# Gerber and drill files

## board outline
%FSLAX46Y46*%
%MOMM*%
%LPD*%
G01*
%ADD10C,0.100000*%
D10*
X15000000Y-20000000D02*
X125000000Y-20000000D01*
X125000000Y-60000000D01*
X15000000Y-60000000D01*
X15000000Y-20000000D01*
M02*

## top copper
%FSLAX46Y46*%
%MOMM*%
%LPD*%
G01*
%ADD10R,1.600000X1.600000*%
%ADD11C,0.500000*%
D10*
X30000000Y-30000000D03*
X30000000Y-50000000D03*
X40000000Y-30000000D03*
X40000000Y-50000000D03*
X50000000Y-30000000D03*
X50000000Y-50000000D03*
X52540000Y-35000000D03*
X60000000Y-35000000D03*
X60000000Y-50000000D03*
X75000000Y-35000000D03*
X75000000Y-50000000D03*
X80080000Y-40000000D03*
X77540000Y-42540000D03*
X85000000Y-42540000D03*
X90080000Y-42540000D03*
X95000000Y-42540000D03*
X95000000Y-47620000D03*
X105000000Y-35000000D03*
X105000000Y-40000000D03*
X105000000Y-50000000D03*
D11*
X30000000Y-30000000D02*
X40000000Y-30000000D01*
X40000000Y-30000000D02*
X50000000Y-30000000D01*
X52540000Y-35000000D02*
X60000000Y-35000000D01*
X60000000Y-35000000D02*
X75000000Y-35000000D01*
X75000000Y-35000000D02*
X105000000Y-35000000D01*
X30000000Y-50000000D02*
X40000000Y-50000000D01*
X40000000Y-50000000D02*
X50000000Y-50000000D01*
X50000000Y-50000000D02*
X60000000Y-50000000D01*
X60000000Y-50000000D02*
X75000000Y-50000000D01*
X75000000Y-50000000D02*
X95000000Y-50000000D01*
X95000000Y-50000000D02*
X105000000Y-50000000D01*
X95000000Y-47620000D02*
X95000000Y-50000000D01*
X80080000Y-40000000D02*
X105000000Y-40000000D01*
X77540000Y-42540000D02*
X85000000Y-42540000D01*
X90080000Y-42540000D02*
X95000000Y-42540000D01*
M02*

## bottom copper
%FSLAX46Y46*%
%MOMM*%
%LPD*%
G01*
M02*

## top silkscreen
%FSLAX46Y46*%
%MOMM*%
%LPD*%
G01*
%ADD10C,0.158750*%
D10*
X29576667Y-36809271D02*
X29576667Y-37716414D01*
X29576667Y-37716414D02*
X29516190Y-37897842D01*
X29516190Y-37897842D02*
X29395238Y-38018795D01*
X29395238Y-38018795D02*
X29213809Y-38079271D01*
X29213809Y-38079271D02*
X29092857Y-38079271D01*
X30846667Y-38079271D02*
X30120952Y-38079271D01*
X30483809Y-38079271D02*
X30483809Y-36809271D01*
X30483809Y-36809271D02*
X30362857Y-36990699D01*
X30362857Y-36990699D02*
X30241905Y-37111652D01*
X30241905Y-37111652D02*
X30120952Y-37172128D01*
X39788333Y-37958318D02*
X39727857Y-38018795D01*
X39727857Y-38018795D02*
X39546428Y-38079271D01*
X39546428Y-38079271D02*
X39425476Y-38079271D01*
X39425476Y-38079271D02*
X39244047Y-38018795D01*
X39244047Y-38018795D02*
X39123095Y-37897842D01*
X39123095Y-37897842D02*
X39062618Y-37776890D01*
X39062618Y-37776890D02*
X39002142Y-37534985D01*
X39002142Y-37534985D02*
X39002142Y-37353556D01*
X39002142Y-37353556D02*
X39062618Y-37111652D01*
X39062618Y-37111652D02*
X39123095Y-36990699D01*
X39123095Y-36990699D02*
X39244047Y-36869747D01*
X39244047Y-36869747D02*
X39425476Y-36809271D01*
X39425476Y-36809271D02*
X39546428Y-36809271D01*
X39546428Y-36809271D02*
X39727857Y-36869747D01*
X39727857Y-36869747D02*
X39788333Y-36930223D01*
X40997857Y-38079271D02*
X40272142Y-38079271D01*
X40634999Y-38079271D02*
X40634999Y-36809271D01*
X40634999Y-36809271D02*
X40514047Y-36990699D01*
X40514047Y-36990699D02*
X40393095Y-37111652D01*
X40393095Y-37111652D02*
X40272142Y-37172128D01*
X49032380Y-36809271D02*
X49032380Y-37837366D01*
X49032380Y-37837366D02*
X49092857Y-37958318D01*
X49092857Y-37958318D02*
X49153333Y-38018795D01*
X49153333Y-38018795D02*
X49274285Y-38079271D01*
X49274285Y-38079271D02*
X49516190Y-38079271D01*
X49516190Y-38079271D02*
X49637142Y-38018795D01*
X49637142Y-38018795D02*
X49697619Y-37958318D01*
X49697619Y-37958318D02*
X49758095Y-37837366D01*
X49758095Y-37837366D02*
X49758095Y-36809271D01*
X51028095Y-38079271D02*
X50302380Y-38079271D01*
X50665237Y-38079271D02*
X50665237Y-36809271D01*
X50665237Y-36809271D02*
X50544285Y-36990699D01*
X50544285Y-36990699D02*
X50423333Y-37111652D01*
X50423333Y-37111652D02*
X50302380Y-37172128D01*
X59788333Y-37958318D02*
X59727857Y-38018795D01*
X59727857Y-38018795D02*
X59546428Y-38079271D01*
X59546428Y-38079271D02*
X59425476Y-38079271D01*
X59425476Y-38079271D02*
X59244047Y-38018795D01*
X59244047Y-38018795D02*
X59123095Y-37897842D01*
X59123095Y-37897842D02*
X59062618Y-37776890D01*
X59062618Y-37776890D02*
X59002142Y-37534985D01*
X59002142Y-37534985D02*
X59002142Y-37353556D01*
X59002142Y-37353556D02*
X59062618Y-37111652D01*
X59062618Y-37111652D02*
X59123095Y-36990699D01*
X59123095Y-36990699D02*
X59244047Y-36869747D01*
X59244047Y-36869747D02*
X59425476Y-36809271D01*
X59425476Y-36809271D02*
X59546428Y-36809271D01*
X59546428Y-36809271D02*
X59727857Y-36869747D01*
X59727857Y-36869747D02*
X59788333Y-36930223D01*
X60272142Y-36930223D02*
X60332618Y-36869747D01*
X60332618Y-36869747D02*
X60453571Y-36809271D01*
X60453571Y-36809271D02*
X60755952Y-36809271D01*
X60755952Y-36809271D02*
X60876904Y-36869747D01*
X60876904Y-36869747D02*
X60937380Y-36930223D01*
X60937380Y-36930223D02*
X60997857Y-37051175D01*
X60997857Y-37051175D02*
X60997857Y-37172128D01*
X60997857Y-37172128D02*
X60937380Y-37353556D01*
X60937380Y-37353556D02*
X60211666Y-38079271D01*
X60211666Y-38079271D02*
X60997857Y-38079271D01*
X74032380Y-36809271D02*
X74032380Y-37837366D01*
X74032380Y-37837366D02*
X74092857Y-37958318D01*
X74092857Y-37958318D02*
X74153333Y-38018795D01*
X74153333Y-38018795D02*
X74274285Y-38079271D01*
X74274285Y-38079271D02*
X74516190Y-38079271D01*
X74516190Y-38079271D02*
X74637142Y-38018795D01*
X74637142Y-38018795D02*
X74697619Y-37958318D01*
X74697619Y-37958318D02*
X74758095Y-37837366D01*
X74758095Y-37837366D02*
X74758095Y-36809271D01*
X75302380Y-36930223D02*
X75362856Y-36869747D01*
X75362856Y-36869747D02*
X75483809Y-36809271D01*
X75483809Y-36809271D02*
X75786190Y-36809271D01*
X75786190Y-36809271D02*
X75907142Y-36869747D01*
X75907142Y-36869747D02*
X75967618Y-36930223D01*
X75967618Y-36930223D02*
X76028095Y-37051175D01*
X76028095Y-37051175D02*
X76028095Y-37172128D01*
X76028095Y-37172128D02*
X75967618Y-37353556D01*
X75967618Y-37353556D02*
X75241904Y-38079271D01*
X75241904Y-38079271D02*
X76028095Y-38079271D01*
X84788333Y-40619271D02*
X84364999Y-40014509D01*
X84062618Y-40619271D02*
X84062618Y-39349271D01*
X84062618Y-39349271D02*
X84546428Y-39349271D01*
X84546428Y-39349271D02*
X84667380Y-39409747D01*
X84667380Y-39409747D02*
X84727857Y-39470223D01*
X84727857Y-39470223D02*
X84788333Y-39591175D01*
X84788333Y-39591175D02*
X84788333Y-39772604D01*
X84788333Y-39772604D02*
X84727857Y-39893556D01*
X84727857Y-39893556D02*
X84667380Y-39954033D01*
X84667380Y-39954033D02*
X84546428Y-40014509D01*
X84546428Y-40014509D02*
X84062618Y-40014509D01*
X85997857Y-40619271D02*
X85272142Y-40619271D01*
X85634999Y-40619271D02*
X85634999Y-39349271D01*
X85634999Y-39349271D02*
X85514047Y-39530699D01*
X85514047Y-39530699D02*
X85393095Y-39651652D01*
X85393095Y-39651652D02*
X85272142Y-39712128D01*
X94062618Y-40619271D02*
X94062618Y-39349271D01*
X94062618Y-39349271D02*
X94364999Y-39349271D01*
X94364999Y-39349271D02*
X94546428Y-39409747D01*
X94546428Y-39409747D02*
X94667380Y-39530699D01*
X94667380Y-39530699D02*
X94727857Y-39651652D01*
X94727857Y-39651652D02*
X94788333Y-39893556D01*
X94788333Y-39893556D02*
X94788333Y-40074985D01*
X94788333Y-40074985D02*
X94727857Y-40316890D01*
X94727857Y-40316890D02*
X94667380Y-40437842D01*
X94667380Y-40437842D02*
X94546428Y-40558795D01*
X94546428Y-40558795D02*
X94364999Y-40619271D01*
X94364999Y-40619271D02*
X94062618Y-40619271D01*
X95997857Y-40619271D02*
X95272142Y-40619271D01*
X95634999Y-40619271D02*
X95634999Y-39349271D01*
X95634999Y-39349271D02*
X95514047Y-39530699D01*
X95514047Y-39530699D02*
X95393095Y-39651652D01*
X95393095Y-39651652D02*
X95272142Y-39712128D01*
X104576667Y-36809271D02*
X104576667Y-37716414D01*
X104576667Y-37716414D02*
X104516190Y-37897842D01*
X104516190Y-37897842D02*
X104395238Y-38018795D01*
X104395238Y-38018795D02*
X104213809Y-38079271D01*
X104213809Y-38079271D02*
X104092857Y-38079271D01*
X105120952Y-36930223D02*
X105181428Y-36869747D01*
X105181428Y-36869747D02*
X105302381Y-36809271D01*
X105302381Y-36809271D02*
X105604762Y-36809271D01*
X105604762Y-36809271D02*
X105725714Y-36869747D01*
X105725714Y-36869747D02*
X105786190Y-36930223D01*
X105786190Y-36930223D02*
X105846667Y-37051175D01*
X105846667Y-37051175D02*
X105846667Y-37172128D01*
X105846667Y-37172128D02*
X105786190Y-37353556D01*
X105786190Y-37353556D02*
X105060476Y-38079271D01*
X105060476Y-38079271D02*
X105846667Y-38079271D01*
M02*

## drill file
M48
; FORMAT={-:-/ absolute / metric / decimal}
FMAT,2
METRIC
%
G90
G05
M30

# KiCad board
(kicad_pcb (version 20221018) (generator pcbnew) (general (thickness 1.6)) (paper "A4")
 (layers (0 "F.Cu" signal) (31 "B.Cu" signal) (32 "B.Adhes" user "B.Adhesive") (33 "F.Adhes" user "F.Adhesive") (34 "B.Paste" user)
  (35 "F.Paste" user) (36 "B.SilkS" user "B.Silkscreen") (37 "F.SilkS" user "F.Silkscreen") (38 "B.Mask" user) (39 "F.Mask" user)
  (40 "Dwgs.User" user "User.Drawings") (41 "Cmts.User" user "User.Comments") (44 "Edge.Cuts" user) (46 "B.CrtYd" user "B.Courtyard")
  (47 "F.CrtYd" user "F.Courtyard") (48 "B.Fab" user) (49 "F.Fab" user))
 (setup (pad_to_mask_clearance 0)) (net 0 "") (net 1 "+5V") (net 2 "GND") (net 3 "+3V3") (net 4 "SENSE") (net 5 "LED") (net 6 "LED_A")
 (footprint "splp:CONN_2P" (layer "F.Cu") (at 30 40)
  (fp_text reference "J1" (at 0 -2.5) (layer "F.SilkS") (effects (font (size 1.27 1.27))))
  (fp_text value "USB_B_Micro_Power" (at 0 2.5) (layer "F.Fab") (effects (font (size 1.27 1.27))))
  (pad "1" smd rect (at 0 -10) (size 1.6 1.6) (layers "F.Cu" "F.Paste" "F.Mask") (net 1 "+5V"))
  (pad "2" smd rect (at 0 10) (size 1.6 1.6) (layers "F.Cu" "F.Paste" "F.Mask") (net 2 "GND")))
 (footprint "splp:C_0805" (layer "F.Cu") (at 40 40)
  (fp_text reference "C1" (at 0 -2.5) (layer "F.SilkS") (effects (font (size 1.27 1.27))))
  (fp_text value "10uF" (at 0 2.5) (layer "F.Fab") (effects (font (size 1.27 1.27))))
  (pad "1" smd rect (at 0 -10) (size 1.6 1.6) (layers "F.Cu" "F.Paste" "F.Mask") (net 1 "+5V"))
  (pad "2" smd rect (at 0 10) (size 1.6 1.6) (layers "F.Cu" "F.Paste" "F.Mask") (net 2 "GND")))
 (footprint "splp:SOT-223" (layer "F.Cu") (at 50 40)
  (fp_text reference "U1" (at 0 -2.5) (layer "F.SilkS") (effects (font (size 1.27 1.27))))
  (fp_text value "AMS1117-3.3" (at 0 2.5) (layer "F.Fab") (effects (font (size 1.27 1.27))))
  (pad "1" smd rect (at 0 -10) (size 1.6 1.6) (layers "F.Cu" "F.Paste" "F.Mask") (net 1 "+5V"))
  (pad "2" smd rect (at 0 10) (size 1.6 1.6) (layers "F.Cu" "F.Paste" "F.Mask") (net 2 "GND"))
  (pad "3" smd rect (at 2.54 -5) (size 1.6 1.6) (layers "F.Cu" "F.Paste" "F.Mask") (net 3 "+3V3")))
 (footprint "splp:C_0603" (layer "F.Cu") (at 60 40)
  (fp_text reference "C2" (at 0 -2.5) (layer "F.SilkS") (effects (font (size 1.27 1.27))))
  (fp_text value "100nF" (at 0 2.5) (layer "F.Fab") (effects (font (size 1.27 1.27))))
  (pad "1" smd rect (at 0 -5) (size 1.6 1.6) (layers "F.Cu" "F.Paste" "F.Mask") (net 3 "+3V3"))
  (pad "2" smd rect (at 0 10) (size 1.6 1.6) (layers "F.Cu" "F.Paste" "F.Mask") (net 2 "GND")))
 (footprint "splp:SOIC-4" (layer "F.Cu") (at 75 40)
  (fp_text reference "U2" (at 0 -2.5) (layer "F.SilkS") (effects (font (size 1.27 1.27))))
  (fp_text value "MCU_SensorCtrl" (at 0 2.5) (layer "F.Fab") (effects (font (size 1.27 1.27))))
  (pad "1" smd rect (at 0 -5) (size 1.6 1.6) (layers "F.Cu" "F.Paste" "F.Mask") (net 3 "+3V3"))
  (pad "2" smd rect (at 0 10) (size 1.6 1.6) (layers "F.Cu" "F.Paste" "F.Mask") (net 2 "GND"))
  (pad "3" smd rect (at 5.08 0) (size 1.6 1.6) (layers "F.Cu" "F.Paste" "F.Mask") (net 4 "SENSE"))
  (pad "4" smd rect (at 2.54 2.54) (size 1.6 1.6) (layers "F.Cu" "F.Paste" "F.Mask") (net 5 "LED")))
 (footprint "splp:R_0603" (layer "F.Cu") (at 85 42.54)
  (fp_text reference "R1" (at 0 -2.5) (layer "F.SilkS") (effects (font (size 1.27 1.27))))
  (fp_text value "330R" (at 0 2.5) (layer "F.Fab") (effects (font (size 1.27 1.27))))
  (pad "1" smd rect (at 0 0) (size 1.6 1.6) (layers "F.Cu" "F.Paste" "F.Mask") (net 5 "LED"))
  (pad "2" smd rect (at 5.08 0) (size 1.6 1.6) (layers "F.Cu" "F.Paste" "F.Mask") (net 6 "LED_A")))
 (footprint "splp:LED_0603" (layer "F.Cu") (at 95 42.54)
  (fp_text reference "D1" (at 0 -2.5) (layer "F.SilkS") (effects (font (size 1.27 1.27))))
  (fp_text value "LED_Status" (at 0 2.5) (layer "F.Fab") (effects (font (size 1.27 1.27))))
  (pad "1" smd rect (at 0 0) (size 1.6 1.6) (layers "F.Cu" "F.Paste" "F.Mask") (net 6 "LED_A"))
  (pad "2" smd rect (at 0 5.08) (size 1.6 1.6) (layers "F.Cu" "F.Paste" "F.Mask") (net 2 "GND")))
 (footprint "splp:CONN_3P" (layer "F.Cu") (at 105 40)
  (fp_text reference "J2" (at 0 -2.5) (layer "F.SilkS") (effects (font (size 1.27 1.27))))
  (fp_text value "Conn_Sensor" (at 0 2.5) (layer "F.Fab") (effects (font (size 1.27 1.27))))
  (pad "1" smd rect (at 0 -5) (size 1.6 1.6) (layers "F.Cu" "F.Paste" "F.Mask") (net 3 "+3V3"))
  (pad "2" smd rect (at 0 0) (size 1.6 1.6) (layers "F.Cu" "F.Paste" "F.Mask") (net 4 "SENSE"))
  (pad "3" smd rect (at 0 10) (size 1.6 1.6) (layers "F.Cu" "F.Paste" "F.Mask") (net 2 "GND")))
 (segment (start 30 30) (end 40 30) (width 0.5) (layer "F.Cu") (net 1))
 (segment (start 40 30) (end 50 30) (width 0.5) (layer "F.Cu") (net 1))
 (segment (start 52.54 35) (end 60 35) (width 0.5) (layer "F.Cu") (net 3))
 (segment (start 60 35) (end 75 35) (width 0.5) (layer "F.Cu") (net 3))
 (segment (start 75 35) (end 105 35) (width 0.5) (layer "F.Cu") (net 3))
 (segment (start 30 50) (end 40 50) (width 0.5) (layer "F.Cu") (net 2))
 (segment (start 40 50) (end 50 50) (width 0.5) (layer "F.Cu") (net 2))
 (segment (start 50 50) (end 60 50) (width 0.5) (layer "F.Cu") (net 2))
 (segment (start 60 50) (end 75 50) (width 0.5) (layer "F.Cu") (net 2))
 (segment (start 75 50) (end 95 50) (width 0.5) (layer "F.Cu") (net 2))
 (segment (start 95 50) (end 105 50) (width 0.5) (layer "F.Cu") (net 2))
 (segment (start 95 47.62) (end 95 50) (width 0.5) (layer "F.Cu") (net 2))
 (segment (start 80.08 40) (end 105 40) (width 0.5) (layer "F.Cu") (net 4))
 (segment (start 77.54 42.54) (end 85 42.54) (width 0.5) (layer "F.Cu") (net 5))
 (segment (start 90.08 42.54) (end 95 42.54) (width 0.5) (layer "F.Cu") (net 6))
 (gr_rect (start 15 20) (end 125 60) (stroke (width 0.1) (type default)) (fill none) (layer "Edge.Cuts")))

